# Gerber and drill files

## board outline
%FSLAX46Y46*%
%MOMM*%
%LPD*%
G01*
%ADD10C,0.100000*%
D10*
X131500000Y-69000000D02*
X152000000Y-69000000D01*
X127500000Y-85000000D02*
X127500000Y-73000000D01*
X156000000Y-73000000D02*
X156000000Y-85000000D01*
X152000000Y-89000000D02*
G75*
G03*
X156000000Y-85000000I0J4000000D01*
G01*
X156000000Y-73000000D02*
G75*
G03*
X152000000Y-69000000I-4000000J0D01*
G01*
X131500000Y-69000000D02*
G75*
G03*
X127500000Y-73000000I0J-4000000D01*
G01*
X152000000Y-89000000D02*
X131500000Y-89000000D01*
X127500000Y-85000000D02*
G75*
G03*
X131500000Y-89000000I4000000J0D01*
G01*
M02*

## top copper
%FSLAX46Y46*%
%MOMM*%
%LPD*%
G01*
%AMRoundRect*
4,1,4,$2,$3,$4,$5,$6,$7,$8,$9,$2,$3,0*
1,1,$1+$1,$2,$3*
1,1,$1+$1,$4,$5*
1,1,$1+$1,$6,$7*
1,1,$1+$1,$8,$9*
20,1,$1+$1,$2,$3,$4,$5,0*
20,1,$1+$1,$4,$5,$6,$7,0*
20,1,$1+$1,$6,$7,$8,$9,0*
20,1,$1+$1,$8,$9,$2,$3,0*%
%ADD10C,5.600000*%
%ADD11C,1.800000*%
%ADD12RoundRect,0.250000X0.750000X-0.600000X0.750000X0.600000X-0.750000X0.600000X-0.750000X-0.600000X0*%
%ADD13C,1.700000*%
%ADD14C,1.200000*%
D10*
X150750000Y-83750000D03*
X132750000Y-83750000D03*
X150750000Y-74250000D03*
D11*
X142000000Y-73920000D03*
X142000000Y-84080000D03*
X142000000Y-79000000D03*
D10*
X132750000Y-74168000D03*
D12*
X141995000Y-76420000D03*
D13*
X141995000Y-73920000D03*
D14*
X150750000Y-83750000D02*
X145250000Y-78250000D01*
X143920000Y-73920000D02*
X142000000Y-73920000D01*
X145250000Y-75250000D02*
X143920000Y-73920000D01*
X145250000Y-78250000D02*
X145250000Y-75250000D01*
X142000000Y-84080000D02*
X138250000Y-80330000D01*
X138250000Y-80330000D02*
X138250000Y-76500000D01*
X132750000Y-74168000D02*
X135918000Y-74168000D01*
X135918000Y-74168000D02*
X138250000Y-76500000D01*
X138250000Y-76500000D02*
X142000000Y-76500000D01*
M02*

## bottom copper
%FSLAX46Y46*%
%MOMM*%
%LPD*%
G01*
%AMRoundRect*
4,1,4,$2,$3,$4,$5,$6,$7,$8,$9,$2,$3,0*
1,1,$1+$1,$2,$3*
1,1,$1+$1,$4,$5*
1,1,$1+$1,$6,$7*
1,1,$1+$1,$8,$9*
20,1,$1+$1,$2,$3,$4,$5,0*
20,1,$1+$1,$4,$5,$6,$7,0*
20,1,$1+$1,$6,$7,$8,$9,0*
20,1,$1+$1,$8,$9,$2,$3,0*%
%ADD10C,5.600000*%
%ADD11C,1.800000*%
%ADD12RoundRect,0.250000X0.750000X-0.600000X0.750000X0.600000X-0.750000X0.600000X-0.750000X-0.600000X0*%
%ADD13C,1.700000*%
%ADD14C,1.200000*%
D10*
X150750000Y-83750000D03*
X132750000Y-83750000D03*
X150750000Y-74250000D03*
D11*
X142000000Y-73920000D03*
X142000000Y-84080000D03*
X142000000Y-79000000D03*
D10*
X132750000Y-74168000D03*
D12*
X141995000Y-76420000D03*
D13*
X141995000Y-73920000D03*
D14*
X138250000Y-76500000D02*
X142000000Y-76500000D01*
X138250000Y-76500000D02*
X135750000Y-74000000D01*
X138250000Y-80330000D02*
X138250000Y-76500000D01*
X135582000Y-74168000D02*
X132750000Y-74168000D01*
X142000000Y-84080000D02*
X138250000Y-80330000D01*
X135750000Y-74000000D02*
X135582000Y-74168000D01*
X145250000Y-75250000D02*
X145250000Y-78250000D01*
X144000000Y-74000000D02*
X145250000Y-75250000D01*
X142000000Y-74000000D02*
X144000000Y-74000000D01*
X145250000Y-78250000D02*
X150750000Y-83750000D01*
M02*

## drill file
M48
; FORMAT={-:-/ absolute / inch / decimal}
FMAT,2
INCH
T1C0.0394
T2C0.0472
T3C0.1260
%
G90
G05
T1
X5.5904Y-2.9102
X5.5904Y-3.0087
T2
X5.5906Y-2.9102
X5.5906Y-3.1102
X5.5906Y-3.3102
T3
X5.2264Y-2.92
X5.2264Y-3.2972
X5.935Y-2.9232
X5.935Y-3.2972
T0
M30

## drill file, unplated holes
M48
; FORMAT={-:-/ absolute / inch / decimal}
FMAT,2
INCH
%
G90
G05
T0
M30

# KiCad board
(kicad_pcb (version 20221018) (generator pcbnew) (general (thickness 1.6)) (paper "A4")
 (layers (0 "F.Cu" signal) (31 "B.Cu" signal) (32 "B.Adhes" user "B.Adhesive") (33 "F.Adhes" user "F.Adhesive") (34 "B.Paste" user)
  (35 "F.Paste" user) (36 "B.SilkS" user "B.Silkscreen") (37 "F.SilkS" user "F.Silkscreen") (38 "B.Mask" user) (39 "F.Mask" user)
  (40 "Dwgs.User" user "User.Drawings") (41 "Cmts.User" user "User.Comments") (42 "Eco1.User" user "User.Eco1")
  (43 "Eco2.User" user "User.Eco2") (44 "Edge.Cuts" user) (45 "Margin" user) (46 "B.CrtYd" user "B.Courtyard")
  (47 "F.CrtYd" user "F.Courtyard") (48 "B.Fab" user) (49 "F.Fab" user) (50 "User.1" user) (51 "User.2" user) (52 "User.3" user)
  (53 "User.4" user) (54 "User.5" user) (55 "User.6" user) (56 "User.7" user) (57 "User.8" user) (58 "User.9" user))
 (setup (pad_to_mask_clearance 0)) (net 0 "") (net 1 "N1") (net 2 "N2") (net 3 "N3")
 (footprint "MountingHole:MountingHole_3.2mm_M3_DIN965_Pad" (layer "F.Cu") (at 150.75 83.75)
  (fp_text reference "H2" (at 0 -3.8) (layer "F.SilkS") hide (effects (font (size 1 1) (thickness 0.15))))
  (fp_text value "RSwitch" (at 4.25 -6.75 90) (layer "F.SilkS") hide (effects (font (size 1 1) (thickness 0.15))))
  (pad "1" thru_hole circle (at 0 0) (size 5.6 5.6) (drill 3.2) (layers "*.Cu" "*.Mask") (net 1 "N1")))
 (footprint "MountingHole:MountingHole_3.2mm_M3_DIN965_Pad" (layer "F.Cu") (at 132.75 83.75)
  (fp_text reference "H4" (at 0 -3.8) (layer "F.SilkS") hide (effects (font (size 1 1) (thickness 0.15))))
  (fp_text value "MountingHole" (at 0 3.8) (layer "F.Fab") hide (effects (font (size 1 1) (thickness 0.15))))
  (pad "1" thru_hole circle (at 0 0) (size 5.6 5.6) (drill 3.2) (layers "*.Cu" "*.Mask")))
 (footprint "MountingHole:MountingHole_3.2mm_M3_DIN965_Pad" (layer "F.Cu") (at 150.75 74.25)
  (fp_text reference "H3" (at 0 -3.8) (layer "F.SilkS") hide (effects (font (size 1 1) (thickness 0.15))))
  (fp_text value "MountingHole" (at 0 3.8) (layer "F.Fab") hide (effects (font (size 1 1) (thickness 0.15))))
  (pad "1" thru_hole circle (at 0 0) (size 5.6 5.6) (drill 3.2) (layers "*.Cu" "*.Mask")))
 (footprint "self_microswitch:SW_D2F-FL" (layer "F.Cu") (at 142 79 90)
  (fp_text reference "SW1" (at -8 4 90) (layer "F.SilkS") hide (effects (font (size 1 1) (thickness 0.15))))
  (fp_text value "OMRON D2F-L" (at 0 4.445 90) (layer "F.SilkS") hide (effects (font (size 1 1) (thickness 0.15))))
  (pad "1" thru_hole circle (at 5.08 0 90) (size 1.8 1.8) (drill 1.2) (layers "*.Cu" "*.Mask") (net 1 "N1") (solder_mask_margin 0.102))
  (pad "2" thru_hole circle (at -5.08 0 90) (size 1.8 1.8) (drill 1.2) (layers "*.Cu" "*.Mask") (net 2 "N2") (solder_mask_margin 0.102))
  (pad "3" thru_hole circle (at 0 0 90) (size 1.8 1.8) (drill 1.2) (layers "*.Cu" "*.Mask") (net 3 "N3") (solder_mask_margin 0.102)))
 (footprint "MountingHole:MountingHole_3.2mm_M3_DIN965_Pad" (layer "F.Cu") (at 132.75 74.168)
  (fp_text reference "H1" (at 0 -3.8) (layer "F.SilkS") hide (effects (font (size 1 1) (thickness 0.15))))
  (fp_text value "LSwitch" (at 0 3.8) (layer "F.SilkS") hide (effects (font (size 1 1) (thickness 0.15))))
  (pad "1" thru_hole circle (at 0 0) (size 5.6 5.6) (drill 3.2) (layers "*.Cu" "*.Mask") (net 2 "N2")))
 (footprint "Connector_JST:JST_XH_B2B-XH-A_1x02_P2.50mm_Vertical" (layer "B.Cu") (at 141.995 76.42 90)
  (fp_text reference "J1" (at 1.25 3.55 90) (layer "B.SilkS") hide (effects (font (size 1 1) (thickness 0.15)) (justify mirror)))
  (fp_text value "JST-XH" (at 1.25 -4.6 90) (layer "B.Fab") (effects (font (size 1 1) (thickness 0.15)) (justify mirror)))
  (pad "1" thru_hole roundrect (at 0 0 90) (size 1.7 2) (drill 1) (layers "*.Cu" "*.Mask") (roundrect_rratio 0.1470588235) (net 2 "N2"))
  (pad "2" thru_hole circle (at 2.5 0 90) (size 1.7 1.7) (drill 1) (layers "*.Cu" "*.Mask") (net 1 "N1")))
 (gr_line (start 131.5 69) (end 152 69) (stroke (width 0.1) (type default)) (layer "Edge.Cuts"))
 (gr_line (start 127.5 85) (end 127.5 73) (stroke (width 0.1) (type default)) (layer "Edge.Cuts"))
 (gr_line (start 156 73) (end 156 85) (stroke (width 0.1) (type default)) (layer "Edge.Cuts"))
 (gr_arc (start 156 85) (mid 154.828427 87.828427) (end 152 89) (stroke (width 0.1) (type default)) (layer "Edge.Cuts"))
 (gr_arc (start 152 69) (mid 154.828427 70.171573) (end 156 73) (stroke (width 0.1) (type default)) (layer "Edge.Cuts"))
 (gr_arc (start 127.5 73) (mid 128.671573 70.171573) (end 131.5 69) (stroke (width 0.1) (type default)) (layer "Edge.Cuts"))
 (gr_line (start 152 89) (end 131.5 89) (stroke (width 0.1) (type default)) (layer "Edge.Cuts"))
 (gr_arc (start 131.5 89) (mid 128.671573 87.828427) (end 127.5 85) (stroke (width 0.1) (type default)) (layer "Edge.Cuts"))
 (segment (start 142 84.08) (end 138.25 80.33) (width 1.2) (layer "F.Cu") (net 2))
 (segment (start 138.25 80.33) (end 138.25 76.5) (width 1.2) (layer "F.Cu") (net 2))
 (segment (start 132.75 74.168) (end 135.918 74.168) (width 1.2) (layer "F.Cu") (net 2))
 (segment (start 135.918 74.168) (end 138.25 76.5) (width 1.2) (layer "F.Cu") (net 2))
 (segment (start 138.25 76.5) (end 142 76.5) (width 1.2) (layer "F.Cu") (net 2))
 (segment (start 138.25 76.5) (end 135.75 74) (width 1.2) (layer "B.Cu") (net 2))
 (segment (start 135.75 74) (end 135.582 74.168) (width 1.2) (layer "B.Cu") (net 2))
 (segment (start 135.582 74.168) (end 132.75 74.168) (width 1.2) (layer "B.Cu") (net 2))
 (segment (start 142 84.08) (end 138.25 80.33) (width 1.2) (layer "B.Cu") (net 2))
 (segment (start 138.25 76.5) (end 142 76.5) (width 1.2) (layer "B.Cu") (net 2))
 (segment (start 138.25 80.33) (end 138.25 76.5) (width 1.2) (layer "B.Cu") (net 2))
 (segment (start 150.75 83.75) (end 145.25 78.25) (width 1.2) (layer "F.Cu") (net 1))
 (segment (start 145.25 75.25) (end 143.92 73.92) (width 1.2) (layer "F.Cu") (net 1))
 (segment (start 143.92 73.92) (end 142 73.92) (width 1.2) (layer "F.Cu") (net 1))
 (segment (start 145.25 78.25) (end 145.25 75.25) (width 1.2) (layer "F.Cu") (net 1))
 (segment (start 145.25 75.25) (end 145.25 78.25) (width 1.2) (layer "B.Cu") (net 1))
 (segment (start 145.25 78.25) (end 150.75 83.75) (width 1.2) (layer "B.Cu") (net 1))
 (segment (start 142 74) (end 144 74) (width 1.2) (layer "B.Cu") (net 1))
 (segment (start 144 74) (end 145.25 75.25) (width 1.2) (layer "B.Cu") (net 1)))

